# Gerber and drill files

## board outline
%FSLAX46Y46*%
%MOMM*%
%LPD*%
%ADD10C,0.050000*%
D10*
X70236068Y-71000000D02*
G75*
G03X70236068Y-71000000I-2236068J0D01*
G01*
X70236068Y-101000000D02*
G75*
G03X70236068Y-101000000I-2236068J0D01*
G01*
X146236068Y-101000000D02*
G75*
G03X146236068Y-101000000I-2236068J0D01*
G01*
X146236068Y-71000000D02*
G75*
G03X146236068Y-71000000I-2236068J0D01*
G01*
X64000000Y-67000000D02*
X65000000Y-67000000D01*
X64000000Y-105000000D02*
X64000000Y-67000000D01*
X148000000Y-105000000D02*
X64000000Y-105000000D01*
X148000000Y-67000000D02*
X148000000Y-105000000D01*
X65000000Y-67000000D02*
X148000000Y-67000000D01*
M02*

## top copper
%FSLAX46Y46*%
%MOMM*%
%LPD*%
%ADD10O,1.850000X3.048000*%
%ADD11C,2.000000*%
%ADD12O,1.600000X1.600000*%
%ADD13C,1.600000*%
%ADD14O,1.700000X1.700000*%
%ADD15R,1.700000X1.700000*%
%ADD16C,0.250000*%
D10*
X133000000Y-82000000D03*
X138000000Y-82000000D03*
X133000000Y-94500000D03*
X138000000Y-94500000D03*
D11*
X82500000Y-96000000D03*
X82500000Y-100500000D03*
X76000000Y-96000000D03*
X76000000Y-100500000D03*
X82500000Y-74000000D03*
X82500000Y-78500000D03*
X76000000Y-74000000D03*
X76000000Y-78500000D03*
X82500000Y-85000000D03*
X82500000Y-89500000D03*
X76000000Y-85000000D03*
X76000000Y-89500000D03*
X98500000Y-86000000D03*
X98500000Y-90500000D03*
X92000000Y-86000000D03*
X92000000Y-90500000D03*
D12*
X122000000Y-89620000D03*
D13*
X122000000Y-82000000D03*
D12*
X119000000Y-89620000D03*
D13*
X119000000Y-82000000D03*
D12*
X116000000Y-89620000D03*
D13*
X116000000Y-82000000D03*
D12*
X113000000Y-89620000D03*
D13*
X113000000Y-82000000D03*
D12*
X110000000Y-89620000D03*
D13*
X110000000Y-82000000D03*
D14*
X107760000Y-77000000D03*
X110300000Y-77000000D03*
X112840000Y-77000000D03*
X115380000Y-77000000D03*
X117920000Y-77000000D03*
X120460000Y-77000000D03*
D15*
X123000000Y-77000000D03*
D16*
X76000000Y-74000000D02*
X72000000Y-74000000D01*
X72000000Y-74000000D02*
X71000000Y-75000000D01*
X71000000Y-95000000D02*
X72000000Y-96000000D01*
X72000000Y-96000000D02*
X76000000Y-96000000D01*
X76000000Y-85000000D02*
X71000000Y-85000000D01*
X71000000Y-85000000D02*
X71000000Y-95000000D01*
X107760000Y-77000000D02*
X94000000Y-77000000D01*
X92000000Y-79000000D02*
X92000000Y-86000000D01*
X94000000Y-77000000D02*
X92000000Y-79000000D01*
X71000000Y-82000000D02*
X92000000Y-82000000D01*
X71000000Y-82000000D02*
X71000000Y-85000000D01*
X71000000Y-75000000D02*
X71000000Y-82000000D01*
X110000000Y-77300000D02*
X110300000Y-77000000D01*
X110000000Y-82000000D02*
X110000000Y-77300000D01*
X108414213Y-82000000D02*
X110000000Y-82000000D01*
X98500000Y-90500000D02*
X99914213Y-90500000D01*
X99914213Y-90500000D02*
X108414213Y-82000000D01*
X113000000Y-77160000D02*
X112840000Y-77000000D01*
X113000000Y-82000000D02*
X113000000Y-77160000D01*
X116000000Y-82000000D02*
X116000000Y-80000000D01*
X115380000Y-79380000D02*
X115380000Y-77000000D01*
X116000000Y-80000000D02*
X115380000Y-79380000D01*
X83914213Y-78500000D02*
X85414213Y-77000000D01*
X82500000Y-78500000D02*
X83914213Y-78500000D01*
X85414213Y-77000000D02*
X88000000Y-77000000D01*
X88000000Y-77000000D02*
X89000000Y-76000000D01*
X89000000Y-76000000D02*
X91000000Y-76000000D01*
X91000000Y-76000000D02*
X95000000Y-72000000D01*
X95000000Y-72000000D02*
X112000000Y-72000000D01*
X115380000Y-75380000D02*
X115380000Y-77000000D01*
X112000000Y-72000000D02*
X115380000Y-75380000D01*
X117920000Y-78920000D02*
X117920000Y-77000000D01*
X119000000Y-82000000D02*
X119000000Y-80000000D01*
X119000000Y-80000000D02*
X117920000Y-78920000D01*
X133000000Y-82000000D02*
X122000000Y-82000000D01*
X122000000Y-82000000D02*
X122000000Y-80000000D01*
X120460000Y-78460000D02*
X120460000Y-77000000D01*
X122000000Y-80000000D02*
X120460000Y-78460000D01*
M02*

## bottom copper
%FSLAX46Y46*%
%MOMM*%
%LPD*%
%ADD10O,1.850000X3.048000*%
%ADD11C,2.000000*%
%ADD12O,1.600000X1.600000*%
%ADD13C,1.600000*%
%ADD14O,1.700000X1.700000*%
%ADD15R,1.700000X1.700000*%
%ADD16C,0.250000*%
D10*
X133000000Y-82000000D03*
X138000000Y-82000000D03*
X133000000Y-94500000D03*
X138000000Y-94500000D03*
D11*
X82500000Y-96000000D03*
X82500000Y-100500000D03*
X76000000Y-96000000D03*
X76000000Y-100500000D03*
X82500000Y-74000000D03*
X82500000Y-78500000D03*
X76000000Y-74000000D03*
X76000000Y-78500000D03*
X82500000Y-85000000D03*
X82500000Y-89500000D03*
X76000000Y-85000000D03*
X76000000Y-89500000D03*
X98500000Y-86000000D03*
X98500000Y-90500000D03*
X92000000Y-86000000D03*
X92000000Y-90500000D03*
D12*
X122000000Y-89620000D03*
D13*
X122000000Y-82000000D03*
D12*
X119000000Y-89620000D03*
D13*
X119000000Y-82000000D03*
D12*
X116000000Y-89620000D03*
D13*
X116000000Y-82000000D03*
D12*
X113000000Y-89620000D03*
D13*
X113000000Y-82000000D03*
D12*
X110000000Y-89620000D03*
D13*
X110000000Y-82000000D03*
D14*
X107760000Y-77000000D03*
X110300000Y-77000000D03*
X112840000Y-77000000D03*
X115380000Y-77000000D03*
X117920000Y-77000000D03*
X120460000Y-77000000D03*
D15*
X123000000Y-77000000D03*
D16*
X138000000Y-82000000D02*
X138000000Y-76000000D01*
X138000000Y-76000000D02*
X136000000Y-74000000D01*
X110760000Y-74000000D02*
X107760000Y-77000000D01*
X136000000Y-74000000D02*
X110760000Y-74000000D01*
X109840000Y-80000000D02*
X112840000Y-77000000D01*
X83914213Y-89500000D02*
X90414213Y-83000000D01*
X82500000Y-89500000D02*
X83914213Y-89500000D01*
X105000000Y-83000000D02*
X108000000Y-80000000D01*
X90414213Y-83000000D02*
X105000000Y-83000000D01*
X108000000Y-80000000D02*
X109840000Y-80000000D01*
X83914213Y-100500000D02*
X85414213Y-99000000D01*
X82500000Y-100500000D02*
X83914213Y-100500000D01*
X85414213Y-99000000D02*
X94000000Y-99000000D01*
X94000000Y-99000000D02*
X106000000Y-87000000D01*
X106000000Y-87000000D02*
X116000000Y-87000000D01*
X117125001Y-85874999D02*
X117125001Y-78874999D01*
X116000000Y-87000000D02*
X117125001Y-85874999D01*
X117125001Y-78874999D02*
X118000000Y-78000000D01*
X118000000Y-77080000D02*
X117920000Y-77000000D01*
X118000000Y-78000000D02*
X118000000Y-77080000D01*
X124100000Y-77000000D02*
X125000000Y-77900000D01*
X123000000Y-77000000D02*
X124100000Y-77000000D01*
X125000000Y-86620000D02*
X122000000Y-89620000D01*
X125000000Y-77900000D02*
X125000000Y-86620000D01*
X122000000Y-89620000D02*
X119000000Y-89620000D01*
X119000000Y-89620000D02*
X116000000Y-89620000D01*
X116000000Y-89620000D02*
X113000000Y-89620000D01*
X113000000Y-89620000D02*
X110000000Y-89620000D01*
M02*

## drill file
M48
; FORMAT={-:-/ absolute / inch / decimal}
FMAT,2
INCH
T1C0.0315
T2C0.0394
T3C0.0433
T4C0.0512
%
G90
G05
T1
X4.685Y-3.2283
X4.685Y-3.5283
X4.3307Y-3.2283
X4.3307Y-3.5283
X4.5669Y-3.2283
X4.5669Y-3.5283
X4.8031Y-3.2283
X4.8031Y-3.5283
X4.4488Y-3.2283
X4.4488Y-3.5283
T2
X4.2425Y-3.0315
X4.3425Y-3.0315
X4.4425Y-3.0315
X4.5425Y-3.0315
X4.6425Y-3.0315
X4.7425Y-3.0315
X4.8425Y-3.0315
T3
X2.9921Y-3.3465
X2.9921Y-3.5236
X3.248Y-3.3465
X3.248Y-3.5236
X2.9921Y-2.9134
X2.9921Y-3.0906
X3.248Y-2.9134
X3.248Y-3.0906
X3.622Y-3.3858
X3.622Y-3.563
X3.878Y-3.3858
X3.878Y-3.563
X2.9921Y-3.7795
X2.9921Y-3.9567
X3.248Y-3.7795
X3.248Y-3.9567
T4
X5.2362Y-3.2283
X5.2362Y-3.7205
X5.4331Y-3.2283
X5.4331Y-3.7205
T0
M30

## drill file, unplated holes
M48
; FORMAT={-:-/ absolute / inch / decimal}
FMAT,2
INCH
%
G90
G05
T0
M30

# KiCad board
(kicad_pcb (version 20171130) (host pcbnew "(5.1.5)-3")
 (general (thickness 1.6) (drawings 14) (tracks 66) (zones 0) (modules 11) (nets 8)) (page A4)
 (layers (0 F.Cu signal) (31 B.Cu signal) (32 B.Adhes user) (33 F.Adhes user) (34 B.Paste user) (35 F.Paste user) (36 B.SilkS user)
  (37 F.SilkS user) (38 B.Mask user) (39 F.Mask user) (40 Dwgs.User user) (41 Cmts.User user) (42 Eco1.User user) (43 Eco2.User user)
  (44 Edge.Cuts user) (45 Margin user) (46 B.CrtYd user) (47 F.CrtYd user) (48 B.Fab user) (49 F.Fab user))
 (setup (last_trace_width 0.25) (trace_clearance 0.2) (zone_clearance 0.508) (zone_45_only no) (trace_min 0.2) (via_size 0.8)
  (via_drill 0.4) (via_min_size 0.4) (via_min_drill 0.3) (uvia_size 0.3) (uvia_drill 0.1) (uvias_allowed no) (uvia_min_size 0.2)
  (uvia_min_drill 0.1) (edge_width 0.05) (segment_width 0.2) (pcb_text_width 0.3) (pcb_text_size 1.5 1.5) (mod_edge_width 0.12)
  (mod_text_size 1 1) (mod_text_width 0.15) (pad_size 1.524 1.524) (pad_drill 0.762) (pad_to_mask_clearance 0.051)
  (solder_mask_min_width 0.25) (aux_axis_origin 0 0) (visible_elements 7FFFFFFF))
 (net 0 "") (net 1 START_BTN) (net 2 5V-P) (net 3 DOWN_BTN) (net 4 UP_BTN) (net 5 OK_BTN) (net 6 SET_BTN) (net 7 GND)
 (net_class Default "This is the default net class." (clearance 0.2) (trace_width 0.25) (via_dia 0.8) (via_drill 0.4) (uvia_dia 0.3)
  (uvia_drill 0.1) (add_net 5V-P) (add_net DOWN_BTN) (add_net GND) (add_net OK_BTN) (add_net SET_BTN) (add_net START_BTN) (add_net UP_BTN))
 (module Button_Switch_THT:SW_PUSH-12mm (layer F.Cu) (at 138 82 270)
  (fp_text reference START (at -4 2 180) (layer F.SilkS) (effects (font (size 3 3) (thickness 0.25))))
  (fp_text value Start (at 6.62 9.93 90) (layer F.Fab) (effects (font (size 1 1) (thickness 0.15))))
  (pad 2 thru_hole oval (at 0 5 270) (size 3.048 1.85) (drill 1.3) (layers *.Cu *.Mask) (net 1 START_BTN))
  (pad 1 thru_hole oval (at 0 0 270) (size 3.048 1.85) (drill 1.3) (layers *.Cu *.Mask) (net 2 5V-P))
  (pad 2 thru_hole oval (at 12.5 5 270) (size 3.048 1.85) (drill 1.3) (layers *.Cu *.Mask) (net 1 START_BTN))
  (pad 1 thru_hole oval (at 12.5 0 270) (size 3.048 1.85) (drill 1.3) (layers *.Cu *.Mask) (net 2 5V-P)))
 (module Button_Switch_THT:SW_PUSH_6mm (layer F.Cu) (at 76 96)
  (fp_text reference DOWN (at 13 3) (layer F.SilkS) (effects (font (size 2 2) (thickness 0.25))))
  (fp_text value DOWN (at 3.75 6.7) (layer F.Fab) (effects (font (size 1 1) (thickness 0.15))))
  (pad 1 thru_hole circle (at 6.5 0 90) (size 2 2) (drill 1.1) (layers *.Cu *.Mask) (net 2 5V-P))
  (pad 2 thru_hole circle (at 6.5 4.5 90) (size 2 2) (drill 1.1) (layers *.Cu *.Mask) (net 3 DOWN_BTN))
  (pad 1 thru_hole circle (at 0 0 90) (size 2 2) (drill 1.1) (layers *.Cu *.Mask) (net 2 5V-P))
  (pad 2 thru_hole circle (at 0 4.5 90) (size 2 2) (drill 1.1) (layers *.Cu *.Mask) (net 3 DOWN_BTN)))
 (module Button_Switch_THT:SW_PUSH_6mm (layer F.Cu) (at 76 74)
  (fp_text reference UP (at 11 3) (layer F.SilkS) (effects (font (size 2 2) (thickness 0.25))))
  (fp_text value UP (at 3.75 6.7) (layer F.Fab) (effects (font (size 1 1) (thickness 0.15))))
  (pad 1 thru_hole circle (at 6.5 0 90) (size 2 2) (drill 1.1) (layers *.Cu *.Mask) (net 2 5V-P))
  (pad 2 thru_hole circle (at 6.5 4.5 90) (size 2 2) (drill 1.1) (layers *.Cu *.Mask) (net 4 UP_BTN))
  (pad 1 thru_hole circle (at 0 0 90) (size 2 2) (drill 1.1) (layers *.Cu *.Mask) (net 2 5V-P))
  (pad 2 thru_hole circle (at 0 4.5 90) (size 2 2) (drill 1.1) (layers *.Cu *.Mask) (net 4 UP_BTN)))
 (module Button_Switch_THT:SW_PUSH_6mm (layer F.Cu) (at 76 85)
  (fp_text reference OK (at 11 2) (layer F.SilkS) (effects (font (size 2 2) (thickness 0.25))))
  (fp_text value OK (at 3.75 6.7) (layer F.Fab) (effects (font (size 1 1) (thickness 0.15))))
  (pad 1 thru_hole circle (at 6.5 0 90) (size 2 2) (drill 1.1) (layers *.Cu *.Mask) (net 2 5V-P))
  (pad 2 thru_hole circle (at 6.5 4.5 90) (size 2 2) (drill 1.1) (layers *.Cu *.Mask) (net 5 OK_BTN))
  (pad 1 thru_hole circle (at 0 0 90) (size 2 2) (drill 1.1) (layers *.Cu *.Mask) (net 2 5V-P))
  (pad 2 thru_hole circle (at 0 4.5 90) (size 2 2) (drill 1.1) (layers *.Cu *.Mask) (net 5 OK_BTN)))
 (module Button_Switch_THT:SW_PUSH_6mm (layer F.Cu) (at 92 86)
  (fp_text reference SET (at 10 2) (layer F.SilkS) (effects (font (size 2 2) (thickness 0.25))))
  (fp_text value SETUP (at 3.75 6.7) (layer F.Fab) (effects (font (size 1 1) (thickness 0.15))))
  (pad 1 thru_hole circle (at 6.5 0 90) (size 2 2) (drill 1.1) (layers *.Cu *.Mask) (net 2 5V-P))
  (pad 2 thru_hole circle (at 6.5 4.5 90) (size 2 2) (drill 1.1) (layers *.Cu *.Mask) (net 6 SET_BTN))
  (pad 1 thru_hole circle (at 0 0 90) (size 2 2) (drill 1.1) (layers *.Cu *.Mask) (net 2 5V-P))
  (pad 2 thru_hole circle (at 0 4.5 90) (size 2 2) (drill 1.1) (layers *.Cu *.Mask) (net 6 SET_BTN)))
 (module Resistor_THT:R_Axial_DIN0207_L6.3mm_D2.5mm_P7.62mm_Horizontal (layer F.Cu) (at 122 82 270)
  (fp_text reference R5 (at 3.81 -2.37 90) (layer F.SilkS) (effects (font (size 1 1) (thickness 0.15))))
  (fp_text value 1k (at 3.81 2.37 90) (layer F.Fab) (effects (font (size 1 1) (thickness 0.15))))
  (pad 2 thru_hole oval (at 7.62 0 270) (size 1.6 1.6) (drill 0.8) (layers *.Cu *.Mask) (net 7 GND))
  (pad 1 thru_hole circle (at 0 0 270) (size 1.6 1.6) (drill 0.8) (layers *.Cu *.Mask) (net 1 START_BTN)))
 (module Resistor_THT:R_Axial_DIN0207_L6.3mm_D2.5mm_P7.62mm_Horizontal (layer F.Cu) (at 119 82 270)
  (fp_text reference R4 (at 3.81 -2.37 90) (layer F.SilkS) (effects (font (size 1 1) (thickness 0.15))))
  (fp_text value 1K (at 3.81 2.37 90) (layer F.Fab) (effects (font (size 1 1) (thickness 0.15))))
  (pad 2 thru_hole oval (at 7.62 0 270) (size 1.6 1.6) (drill 0.8) (layers *.Cu *.Mask) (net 7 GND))
  (pad 1 thru_hole circle (at 0 0 270) (size 1.6 1.6) (drill 0.8) (layers *.Cu *.Mask) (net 3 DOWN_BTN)))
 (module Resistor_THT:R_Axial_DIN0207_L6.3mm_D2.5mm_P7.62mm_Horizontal (layer F.Cu) (at 116 82 270)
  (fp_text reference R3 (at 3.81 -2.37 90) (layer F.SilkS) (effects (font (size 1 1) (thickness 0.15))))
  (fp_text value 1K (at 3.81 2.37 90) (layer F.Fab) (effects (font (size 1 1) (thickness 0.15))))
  (pad 2 thru_hole oval (at 7.62 0 270) (size 1.6 1.6) (drill 0.8) (layers *.Cu *.Mask) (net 7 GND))
  (pad 1 thru_hole circle (at 0 0 270) (size 1.6 1.6) (drill 0.8) (layers *.Cu *.Mask) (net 4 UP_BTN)))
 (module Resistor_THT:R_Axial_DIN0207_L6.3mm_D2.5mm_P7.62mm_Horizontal (layer F.Cu) (at 113 82 270)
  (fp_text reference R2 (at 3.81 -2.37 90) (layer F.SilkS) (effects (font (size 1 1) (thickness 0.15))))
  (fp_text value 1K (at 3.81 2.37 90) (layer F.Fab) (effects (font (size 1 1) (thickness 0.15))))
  (pad 2 thru_hole oval (at 7.62 0 270) (size 1.6 1.6) (drill 0.8) (layers *.Cu *.Mask) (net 7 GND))
  (pad 1 thru_hole circle (at 0 0 270) (size 1.6 1.6) (drill 0.8) (layers *.Cu *.Mask) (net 5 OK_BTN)))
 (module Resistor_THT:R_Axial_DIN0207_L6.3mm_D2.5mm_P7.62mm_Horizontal (layer F.Cu) (at 110 82 270)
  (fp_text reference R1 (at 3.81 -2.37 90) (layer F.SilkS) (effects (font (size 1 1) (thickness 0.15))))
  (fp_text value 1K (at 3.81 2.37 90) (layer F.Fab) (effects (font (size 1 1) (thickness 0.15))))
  (pad 2 thru_hole oval (at 7.62 0 270) (size 1.6 1.6) (drill 0.8) (layers *.Cu *.Mask) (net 7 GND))
  (pad 1 thru_hole circle (at 0 0 270) (size 1.6 1.6) (drill 0.8) (layers *.Cu *.Mask) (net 6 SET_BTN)))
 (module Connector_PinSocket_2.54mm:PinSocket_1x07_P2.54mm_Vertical (layer F.Cu) (at 123 77 270)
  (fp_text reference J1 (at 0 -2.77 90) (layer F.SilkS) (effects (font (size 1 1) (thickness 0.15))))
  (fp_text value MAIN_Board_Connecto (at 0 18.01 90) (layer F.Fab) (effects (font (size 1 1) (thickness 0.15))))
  (pad 7 thru_hole oval (at 0 15.24 270) (size 1.7 1.7) (drill 1) (layers *.Cu *.Mask) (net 2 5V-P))
  (pad 6 thru_hole oval (at 0 12.7 270) (size 1.7 1.7) (drill 1) (layers *.Cu *.Mask) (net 6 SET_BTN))
  (pad 5 thru_hole oval (at 0 10.16 270) (size 1.7 1.7) (drill 1) (layers *.Cu *.Mask) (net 5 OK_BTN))
  (pad 4 thru_hole oval (at 0 7.62 270) (size 1.7 1.7) (drill 1) (layers *.Cu *.Mask) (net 4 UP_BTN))
  (pad 3 thru_hole oval (at 0 5.08 270) (size 1.7 1.7) (drill 1) (layers *.Cu *.Mask) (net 3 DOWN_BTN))
  (pad 2 thru_hole oval (at 0 2.54 270) (size 1.7 1.7) (drill 1) (layers *.Cu *.Mask) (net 1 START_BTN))
  (pad 1 thru_hole rect (at 0 0 270) (size 1.7 1.7) (drill 1) (layers *.Cu *.Mask) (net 7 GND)))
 (gr_circle (center 68 71) (end 70 72) (layer Edge.Cuts) (width 0.05))
 (gr_circle (center 68 101) (end 70 102) (layer Edge.Cuts) (width 0.05))
 (gr_circle (center 144 101) (end 146 102) (layer Edge.Cuts) (width 0.05))
 (gr_circle (center 144 71) (end 146 72) (layer Edge.Cuts) (width 0.05))
 (gr_line (start 64 67) (end 65 67) (layer Edge.Cuts) (width 0.05))
 (gr_line (start 64 105) (end 64 67) (layer Edge.Cuts) (width 0.05))
 (gr_line (start 148 105) (end 64 105) (layer Edge.Cuts) (width 0.05))
 (gr_line (start 148 67) (end 148 105) (layer Edge.Cuts) (width 0.05))
 (gr_line (start 65 67) (end 148 67) (layer Edge.Cuts) (width 0.05))
 (segment (start 76 74) (end 72 74) (width 0.25) (layer F.Cu) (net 2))
 (segment (start 72 74) (end 71 75) (width 0.25) (layer F.Cu) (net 2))
 (segment (start 71 95) (end 72 96) (width 0.25) (layer F.Cu) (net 2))
 (segment (start 72 96) (end 76 96) (width 0.25) (layer F.Cu) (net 2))
 (segment (start 76 85) (end 71 85) (width 0.25) (layer F.Cu) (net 2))
 (segment (start 71 85) (end 71 95) (width 0.25) (layer F.Cu) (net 2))
 (segment (start 107.76 77) (end 94 77) (width 0.25) (layer F.Cu) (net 2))
 (segment (start 92 79) (end 92 86) (width 0.25) (layer F.Cu) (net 2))
 (segment (start 94 77) (end 92 79) (width 0.25) (layer F.Cu) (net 2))
 (segment (start 71 82) (end 92 82) (width 0.25) (layer F.Cu) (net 2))
 (segment (start 71 82) (end 71 85) (width 0.25) (layer F.Cu) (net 2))
 (segment (start 71 75) (end 71 82) (width 0.25) (layer F.Cu) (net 2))
 (segment (start 138 82) (end 138 76) (width 0.25) (layer B.Cu) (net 2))
 (segment (start 138 76) (end 136 74) (width 0.25) (layer B.Cu) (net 2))
 (segment (start 110.76 74) (end 107.76 77) (width 0.25) (layer B.Cu) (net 2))
 (segment (start 136 74) (end 110.76 74) (width 0.25) (layer B.Cu) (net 2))
 (segment (start 110 77.3) (end 110.3 77) (width 0.25) (layer F.Cu) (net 6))
 (segment (start 110 82) (end 110 77.3) (width 0.25) (layer F.Cu) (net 6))
 (segment (start 108.414213 82) (end 110 82) (width 0.25) (layer F.Cu) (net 6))
 (segment (start 98.5 90.5) (end 99.914213 90.5) (width 0.25) (layer F.Cu) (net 6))
 (segment (start 99.914213 90.5) (end 108.414213 82) (width 0.25) (layer F.Cu) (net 6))
 (segment (start 113 77.16) (end 112.84 77) (width 0.25) (layer F.Cu) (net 5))
 (segment (start 113 82) (end 113 77.16) (width 0.25) (layer F.Cu) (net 5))
 (segment (start 109.84 80) (end 112.84 77) (width 0.25) (layer B.Cu) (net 5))
 (segment (start 83.914213 89.5) (end 90.414213 83) (width 0.25) (layer B.Cu) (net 5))
 (segment (start 82.5 89.5) (end 83.914213 89.5) (width 0.25) (layer B.Cu) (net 5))
 (segment (start 105 83) (end 108 80) (width 0.25) (layer B.Cu) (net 5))
 (segment (start 90.414213 83) (end 105 83) (width 0.25) (layer B.Cu) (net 5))
 (segment (start 108 80) (end 109.84 80) (width 0.25) (layer B.Cu) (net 5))
 (segment (start 116 82) (end 116 80) (width 0.25) (layer F.Cu) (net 4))
 (segment (start 115.38 79.38) (end 115.38 77) (width 0.25) (layer F.Cu) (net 4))
 (segment (start 116 80) (end 115.38 79.38) (width 0.25) (layer F.Cu) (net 4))
 (segment (start 83.914213 78.5) (end 85.414213 77) (width 0.25) (layer F.Cu) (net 4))
 (segment (start 82.5 78.5) (end 83.914213 78.5) (width 0.25) (layer F.Cu) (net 4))
 (segment (start 85.414213 77) (end 88 77) (width 0.25) (layer F.Cu) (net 4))
 (segment (start 88 77) (end 89 76) (width 0.25) (layer F.Cu) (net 4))
 (segment (start 89 76) (end 91 76) (width 0.25) (layer F.Cu) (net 4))
 (segment (start 91 76) (end 95 72) (width 0.25) (layer F.Cu) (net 4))
 (segment (start 95 72) (end 112 72) (width 0.25) (layer F.Cu) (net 4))
 (segment (start 115.38 75.38) (end 115.38 77) (width 0.25) (layer F.Cu) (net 4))
 (segment (start 112 72) (end 115.38 75.38) (width 0.25) (layer F.Cu) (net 4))
 (segment (start 117.92 78.92) (end 117.92 77) (width 0.25) (layer F.Cu) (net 3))
 (segment (start 119 82) (end 119 80) (width 0.25) (layer F.Cu) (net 3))
 (segment (start 119 80) (end 117.92 78.92) (width 0.25) (layer F.Cu) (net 3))
 (segment (start 83.914213 100.5) (end 85.414213 99) (width 0.25) (layer B.Cu) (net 3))
 (segment (start 82.5 100.5) (end 83.914213 100.5) (width 0.25) (layer B.Cu) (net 3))
 (segment (start 85.414213 99) (end 94 99) (width 0.25) (layer B.Cu) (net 3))
 (segment (start 94 99) (end 106 87) (width 0.25) (layer B.Cu) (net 3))
 (segment (start 106 87) (end 116 87) (width 0.25) (layer B.Cu) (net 3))
 (segment (start 117.125001 85.874999) (end 117.125001 78.874999) (width 0.25) (layer B.Cu) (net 3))
 (segment (start 116 87) (end 117.125001 85.874999) (width 0.25) (layer B.Cu) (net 3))
 (segment (start 117.125001 78.874999) (end 118 78) (width 0.25) (layer B.Cu) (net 3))
 (segment (start 118 77.08) (end 117.92 77) (width 0.25) (layer B.Cu) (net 3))
 (segment (start 118 78) (end 118 77.08) (width 0.25) (layer B.Cu) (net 3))
 (segment (start 133 82) (end 122 82) (width 0.25) (layer F.Cu) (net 1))
 (segment (start 122 82) (end 122 80) (width 0.25) (layer F.Cu) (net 1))
 (segment (start 120.46 78.46) (end 120.46 77) (width 0.25) (layer F.Cu) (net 1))
 (segment (start 122 80) (end 120.46 78.46) (width 0.25) (layer F.Cu) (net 1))
 (segment (start 124.1 77) (end 125 77.9) (width 0.25) (layer B.Cu) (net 7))
 (segment (start 123 77) (end 124.1 77) (width 0.25) (layer B.Cu) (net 7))
 (segment (start 125 86.62) (end 122 89.62) (width 0.25) (layer B.Cu) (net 7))
 (segment (start 125 77.9) (end 125 86.62) (width 0.25) (layer B.Cu) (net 7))
 (segment (start 122 89.62) (end 119 89.62) (width 0.25) (layer B.Cu) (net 7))
 (segment (start 119 89.62) (end 116 89.62) (width 0.25) (layer B.Cu) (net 7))
 (segment (start 116 89.62) (end 113 89.62) (width 0.25) (layer B.Cu) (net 7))
 (segment (start 113 89.62) (end 110 89.62) (width 0.25) (layer B.Cu) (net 7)))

